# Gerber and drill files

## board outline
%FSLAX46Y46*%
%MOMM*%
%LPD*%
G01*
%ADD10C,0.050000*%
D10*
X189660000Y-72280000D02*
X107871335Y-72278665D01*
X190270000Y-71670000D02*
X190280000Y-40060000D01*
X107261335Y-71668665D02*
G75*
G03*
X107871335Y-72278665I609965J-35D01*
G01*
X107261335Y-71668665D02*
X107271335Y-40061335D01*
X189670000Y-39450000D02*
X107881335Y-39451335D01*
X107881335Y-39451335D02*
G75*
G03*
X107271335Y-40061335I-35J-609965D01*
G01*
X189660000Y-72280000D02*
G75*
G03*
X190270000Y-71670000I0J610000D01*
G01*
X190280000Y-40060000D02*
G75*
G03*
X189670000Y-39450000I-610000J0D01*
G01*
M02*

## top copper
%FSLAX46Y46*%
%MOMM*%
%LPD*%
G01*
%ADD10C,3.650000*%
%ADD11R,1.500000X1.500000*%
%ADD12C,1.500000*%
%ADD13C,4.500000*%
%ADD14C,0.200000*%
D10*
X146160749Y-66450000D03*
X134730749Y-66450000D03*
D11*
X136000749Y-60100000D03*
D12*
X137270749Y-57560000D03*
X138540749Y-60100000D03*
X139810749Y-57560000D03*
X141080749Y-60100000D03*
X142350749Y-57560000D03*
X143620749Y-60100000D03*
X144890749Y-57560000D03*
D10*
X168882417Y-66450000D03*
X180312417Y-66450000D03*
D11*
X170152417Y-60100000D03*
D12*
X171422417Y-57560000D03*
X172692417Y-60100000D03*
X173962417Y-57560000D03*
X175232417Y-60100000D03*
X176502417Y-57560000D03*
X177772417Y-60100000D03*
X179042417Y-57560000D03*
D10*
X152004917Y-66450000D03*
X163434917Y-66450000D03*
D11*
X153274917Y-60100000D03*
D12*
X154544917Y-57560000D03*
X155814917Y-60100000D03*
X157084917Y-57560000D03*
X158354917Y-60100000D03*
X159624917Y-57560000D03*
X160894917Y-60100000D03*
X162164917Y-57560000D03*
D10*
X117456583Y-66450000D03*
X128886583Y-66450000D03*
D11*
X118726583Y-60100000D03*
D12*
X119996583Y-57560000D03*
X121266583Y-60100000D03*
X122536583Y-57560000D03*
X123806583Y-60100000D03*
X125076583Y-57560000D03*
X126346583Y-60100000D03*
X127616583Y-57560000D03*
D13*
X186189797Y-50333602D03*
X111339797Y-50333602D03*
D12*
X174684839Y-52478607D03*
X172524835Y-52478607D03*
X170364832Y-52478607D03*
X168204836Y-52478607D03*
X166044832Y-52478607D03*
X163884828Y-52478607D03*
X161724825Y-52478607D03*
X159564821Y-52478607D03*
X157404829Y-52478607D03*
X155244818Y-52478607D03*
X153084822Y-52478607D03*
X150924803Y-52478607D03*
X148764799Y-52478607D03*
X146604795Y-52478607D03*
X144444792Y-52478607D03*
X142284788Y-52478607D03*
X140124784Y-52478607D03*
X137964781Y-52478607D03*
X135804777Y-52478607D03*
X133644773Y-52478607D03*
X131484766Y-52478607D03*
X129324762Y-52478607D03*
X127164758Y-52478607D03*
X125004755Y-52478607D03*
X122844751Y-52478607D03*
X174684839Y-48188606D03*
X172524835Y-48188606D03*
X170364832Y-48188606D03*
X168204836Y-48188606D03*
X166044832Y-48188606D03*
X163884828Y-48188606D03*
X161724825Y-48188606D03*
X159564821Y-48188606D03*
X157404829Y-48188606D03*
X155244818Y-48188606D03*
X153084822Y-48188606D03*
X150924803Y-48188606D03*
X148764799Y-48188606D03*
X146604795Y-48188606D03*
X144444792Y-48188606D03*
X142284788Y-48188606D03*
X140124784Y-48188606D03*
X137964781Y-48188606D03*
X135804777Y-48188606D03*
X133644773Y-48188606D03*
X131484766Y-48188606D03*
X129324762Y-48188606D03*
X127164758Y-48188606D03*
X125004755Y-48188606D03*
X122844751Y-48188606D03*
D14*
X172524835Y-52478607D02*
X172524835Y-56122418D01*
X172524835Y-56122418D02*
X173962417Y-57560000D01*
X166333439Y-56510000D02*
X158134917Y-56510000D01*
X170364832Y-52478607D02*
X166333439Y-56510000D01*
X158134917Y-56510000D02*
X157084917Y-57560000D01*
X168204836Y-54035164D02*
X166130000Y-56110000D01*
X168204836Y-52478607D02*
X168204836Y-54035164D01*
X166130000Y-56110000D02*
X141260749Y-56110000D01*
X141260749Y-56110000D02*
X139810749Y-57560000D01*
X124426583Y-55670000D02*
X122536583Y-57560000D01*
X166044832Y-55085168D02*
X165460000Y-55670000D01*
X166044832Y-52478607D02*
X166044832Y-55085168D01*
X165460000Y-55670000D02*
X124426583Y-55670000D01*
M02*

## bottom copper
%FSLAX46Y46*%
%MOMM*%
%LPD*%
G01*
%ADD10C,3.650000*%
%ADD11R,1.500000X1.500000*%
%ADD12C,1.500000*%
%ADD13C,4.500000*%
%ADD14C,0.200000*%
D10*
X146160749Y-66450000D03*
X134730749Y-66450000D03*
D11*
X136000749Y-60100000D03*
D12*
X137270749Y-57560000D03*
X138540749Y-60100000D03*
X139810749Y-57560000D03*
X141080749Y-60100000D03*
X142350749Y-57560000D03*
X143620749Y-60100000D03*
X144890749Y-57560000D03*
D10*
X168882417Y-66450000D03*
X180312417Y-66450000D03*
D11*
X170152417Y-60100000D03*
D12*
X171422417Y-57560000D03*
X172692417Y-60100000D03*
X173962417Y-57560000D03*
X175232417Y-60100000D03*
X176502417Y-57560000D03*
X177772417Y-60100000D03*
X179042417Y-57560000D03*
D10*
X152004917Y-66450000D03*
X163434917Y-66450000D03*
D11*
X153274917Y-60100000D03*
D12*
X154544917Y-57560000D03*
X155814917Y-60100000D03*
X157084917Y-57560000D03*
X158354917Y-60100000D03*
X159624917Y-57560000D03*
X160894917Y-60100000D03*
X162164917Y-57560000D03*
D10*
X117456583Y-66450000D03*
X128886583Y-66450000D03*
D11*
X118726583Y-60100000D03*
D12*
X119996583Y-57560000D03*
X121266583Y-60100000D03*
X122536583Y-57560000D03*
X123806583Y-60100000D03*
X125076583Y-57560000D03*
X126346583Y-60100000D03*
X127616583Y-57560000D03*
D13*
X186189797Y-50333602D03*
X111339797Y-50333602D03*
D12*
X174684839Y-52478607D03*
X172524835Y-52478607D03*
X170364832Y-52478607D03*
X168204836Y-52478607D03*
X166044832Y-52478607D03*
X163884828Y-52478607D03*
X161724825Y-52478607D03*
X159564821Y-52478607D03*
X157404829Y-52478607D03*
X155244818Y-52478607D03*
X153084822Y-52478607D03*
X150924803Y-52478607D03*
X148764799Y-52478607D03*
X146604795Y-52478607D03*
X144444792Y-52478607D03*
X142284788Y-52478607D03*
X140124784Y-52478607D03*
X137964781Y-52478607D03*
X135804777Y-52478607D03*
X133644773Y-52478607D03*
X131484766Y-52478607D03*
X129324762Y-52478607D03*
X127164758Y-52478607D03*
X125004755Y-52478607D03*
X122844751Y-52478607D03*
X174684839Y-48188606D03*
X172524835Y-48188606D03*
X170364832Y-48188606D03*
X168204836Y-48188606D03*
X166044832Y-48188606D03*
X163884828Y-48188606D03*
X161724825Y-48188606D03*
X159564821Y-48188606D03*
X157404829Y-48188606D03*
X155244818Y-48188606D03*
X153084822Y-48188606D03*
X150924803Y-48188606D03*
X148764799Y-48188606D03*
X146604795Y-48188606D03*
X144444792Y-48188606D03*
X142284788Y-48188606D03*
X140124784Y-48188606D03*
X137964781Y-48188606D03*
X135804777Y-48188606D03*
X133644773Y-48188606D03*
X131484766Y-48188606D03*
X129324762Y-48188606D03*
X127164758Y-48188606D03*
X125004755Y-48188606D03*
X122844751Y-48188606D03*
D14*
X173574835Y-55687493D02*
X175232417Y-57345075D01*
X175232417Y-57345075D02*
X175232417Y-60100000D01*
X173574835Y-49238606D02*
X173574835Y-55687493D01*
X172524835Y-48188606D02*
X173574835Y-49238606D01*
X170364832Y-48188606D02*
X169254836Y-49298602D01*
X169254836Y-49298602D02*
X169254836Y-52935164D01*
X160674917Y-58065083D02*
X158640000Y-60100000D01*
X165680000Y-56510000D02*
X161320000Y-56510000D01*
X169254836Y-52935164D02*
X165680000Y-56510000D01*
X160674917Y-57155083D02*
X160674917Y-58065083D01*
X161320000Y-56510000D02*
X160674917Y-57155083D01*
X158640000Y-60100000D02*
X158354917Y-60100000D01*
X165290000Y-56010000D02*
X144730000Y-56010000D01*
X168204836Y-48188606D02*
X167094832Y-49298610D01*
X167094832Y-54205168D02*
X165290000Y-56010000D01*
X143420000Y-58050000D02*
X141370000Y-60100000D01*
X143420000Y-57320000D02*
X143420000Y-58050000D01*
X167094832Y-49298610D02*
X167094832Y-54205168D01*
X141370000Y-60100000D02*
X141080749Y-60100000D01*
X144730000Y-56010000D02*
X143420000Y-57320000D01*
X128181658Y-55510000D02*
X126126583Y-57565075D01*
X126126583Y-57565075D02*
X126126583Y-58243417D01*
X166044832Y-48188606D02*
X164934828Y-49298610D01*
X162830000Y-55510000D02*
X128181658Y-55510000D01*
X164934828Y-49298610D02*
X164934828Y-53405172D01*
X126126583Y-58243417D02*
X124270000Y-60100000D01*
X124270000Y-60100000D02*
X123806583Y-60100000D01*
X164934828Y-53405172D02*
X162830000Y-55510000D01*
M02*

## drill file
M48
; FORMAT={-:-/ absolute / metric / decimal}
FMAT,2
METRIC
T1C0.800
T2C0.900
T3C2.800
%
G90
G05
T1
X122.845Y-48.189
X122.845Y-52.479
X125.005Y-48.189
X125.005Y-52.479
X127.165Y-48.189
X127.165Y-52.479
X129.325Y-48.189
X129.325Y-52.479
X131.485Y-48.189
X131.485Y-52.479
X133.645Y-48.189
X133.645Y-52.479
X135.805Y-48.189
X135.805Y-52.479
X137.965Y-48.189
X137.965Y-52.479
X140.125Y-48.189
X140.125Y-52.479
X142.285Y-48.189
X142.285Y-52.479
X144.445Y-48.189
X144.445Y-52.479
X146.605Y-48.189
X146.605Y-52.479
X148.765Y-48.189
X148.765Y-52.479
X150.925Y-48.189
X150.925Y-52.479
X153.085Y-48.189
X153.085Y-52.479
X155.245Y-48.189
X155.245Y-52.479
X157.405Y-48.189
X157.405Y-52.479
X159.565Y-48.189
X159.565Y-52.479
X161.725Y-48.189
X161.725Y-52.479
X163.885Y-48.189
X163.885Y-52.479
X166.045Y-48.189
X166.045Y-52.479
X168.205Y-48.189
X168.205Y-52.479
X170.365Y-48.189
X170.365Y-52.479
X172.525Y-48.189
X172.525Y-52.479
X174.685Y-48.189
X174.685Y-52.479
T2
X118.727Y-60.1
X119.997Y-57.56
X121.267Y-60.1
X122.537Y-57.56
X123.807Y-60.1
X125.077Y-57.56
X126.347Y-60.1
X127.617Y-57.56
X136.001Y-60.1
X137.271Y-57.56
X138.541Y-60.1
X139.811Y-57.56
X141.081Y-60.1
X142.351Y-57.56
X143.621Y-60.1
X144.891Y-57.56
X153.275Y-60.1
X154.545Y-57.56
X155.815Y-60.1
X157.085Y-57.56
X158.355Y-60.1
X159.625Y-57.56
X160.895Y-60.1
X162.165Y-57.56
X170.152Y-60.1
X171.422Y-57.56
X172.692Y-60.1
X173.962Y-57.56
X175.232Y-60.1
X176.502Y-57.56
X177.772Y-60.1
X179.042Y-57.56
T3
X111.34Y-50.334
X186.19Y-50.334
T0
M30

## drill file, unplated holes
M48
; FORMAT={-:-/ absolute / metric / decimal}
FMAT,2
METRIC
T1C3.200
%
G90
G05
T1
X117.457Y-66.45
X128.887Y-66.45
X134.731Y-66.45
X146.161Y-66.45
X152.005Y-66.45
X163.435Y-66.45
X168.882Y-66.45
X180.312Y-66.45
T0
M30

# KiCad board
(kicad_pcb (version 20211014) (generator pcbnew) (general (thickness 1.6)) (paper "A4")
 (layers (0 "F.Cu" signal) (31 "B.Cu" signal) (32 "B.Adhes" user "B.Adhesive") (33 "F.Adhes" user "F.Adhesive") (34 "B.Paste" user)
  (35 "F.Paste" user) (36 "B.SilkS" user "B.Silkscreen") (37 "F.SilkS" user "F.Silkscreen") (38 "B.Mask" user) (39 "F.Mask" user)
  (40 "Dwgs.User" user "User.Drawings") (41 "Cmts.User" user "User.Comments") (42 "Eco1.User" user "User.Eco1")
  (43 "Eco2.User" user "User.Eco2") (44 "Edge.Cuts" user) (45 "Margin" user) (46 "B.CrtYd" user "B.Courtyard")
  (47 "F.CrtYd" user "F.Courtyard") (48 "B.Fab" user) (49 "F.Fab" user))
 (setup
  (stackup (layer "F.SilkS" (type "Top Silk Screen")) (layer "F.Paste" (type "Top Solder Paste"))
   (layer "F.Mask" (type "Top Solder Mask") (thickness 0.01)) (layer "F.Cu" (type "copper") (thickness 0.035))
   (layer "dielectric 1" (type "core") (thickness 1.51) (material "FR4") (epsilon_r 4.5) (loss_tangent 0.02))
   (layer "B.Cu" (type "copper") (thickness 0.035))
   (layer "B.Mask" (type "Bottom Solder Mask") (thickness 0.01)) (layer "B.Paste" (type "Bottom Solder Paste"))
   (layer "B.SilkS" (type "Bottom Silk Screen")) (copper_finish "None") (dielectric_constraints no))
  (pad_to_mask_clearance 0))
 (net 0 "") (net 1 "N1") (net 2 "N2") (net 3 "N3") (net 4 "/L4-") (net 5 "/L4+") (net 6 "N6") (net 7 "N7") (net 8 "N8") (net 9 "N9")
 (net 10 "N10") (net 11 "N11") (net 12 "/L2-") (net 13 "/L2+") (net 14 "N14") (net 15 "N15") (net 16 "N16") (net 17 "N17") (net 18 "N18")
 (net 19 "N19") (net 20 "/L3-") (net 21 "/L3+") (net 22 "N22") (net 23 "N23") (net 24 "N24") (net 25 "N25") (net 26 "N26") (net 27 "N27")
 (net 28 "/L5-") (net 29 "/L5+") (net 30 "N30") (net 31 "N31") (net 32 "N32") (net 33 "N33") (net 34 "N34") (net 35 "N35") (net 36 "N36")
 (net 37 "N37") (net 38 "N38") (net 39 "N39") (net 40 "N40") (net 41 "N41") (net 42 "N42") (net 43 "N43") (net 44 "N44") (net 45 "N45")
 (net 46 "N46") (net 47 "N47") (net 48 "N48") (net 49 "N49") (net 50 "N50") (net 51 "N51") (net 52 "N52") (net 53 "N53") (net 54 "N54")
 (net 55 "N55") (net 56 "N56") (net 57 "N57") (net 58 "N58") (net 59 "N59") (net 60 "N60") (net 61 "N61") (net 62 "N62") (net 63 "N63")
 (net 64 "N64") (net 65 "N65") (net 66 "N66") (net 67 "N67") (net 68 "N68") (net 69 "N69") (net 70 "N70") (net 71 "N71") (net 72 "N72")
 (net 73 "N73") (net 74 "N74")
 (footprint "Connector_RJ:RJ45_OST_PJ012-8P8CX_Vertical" (layer "F.Cu") (at 136.000749 60.1)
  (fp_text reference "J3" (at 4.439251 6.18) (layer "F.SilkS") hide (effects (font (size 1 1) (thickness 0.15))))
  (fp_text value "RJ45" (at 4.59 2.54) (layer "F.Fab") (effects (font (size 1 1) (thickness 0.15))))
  (pad "" np_thru_hole circle (at 10.16 6.35) (size 3.65 3.65) (drill 3.2) (layers F&B.Cu *.SilkS *.Mask))
  (pad "" np_thru_hole circle (at -1.27 6.35) (size 3.65 3.65) (drill 3.2) (layers F&B.Cu *.SilkS *.Mask))
  (pad "1" thru_hole rect (at 0 0) (size 1.5 1.5) (drill 0.9) (layers *.Cu *.Mask) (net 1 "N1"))
  (pad "2" thru_hole circle (at 1.27 -2.54) (size 1.5 1.5) (drill 0.9) (layers *.Cu *.Mask) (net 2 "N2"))
  (pad "3" thru_hole circle (at 2.54 0) (size 1.5 1.5) (drill 0.9) (layers *.Cu *.Mask) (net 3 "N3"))
  (pad "4" thru_hole circle (at 3.81 -2.54) (size 1.5 1.5) (drill 0.9) (layers *.Cu *.Mask) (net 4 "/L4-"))
  (pad "5" thru_hole circle (at 5.08 0) (size 1.5 1.5) (drill 0.9) (layers *.Cu *.Mask) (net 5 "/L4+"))
  (pad "6" thru_hole circle (at 6.35 -2.54) (size 1.5 1.5) (drill 0.9) (layers *.Cu *.Mask) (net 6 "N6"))
  (pad "7" thru_hole circle (at 7.62 0) (size 1.5 1.5) (drill 0.9) (layers *.Cu *.Mask) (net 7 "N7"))
  (pad "8" thru_hole circle (at 8.89 -2.54) (size 1.5 1.5) (drill 0.9) (layers *.Cu *.Mask) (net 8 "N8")))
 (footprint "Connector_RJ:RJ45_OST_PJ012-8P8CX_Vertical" (layer "F.Cu") (at 170.152417 60.1)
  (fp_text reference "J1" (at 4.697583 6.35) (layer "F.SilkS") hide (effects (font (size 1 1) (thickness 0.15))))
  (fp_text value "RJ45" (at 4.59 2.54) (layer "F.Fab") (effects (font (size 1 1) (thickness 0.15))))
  (pad "" np_thru_hole circle (at -1.27 6.35) (size 3.65 3.65) (drill 3.2) (layers F&B.Cu *.SilkS *.Mask))
  (pad "" np_thru_hole circle (at 10.16 6.35) (size 3.65 3.65) (drill 3.2) (layers F&B.Cu *.SilkS *.Mask))
  (pad "1" thru_hole rect (at 0 0) (size 1.5 1.5) (drill 0.9) (layers *.Cu *.Mask) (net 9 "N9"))
  (pad "2" thru_hole circle (at 1.27 -2.54) (size 1.5 1.5) (drill 0.9) (layers *.Cu *.Mask) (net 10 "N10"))
  (pad "3" thru_hole circle (at 2.54 0) (size 1.5 1.5) (drill 0.9) (layers *.Cu *.Mask) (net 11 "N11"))
  (pad "4" thru_hole circle (at 3.81 -2.54) (size 1.5 1.5) (drill 0.9) (layers *.Cu *.Mask) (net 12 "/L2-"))
  (pad "5" thru_hole circle (at 5.08 0) (size 1.5 1.5) (drill 0.9) (layers *.Cu *.Mask) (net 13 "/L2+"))
  (pad "6" thru_hole circle (at 6.35 -2.54) (size 1.5 1.5) (drill 0.9) (layers *.Cu *.Mask) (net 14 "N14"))
  (pad "7" thru_hole circle (at 7.62 0) (size 1.5 1.5) (drill 0.9) (layers *.Cu *.Mask) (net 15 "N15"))
  (pad "8" thru_hole circle (at 8.89 -2.54) (size 1.5 1.5) (drill 0.9) (layers *.Cu *.Mask) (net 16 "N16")))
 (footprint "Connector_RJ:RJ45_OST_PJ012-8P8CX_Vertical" (layer "F.Cu") (at 153.274917 60.1)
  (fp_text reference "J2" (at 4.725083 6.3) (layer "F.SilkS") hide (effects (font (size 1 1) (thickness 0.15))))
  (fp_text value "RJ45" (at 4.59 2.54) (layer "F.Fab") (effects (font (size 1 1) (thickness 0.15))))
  (pad "" np_thru_hole circle (at -1.27 6.35) (size 3.65 3.65) (drill 3.2) (layers F&B.Cu *.SilkS *.Mask))
  (pad "" np_thru_hole circle (at 10.16 6.35) (size 3.65 3.65) (drill 3.2) (layers F&B.Cu *.SilkS *.Mask))
  (pad "1" thru_hole rect (at 0 0) (size 1.5 1.5) (drill 0.9) (layers *.Cu *.Mask) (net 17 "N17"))
  (pad "2" thru_hole circle (at 1.27 -2.54) (size 1.5 1.5) (drill 0.9) (layers *.Cu *.Mask) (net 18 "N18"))
  (pad "3" thru_hole circle (at 2.54 0) (size 1.5 1.5) (drill 0.9) (layers *.Cu *.Mask) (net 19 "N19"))
  (pad "4" thru_hole circle (at 3.81 -2.54) (size 1.5 1.5) (drill 0.9) (layers *.Cu *.Mask) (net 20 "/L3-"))
  (pad "5" thru_hole circle (at 5.08 0) (size 1.5 1.5) (drill 0.9) (layers *.Cu *.Mask) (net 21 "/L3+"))
  (pad "6" thru_hole circle (at 6.35 -2.54) (size 1.5 1.5) (drill 0.9) (layers *.Cu *.Mask) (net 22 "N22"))
  (pad "7" thru_hole circle (at 7.62 0) (size 1.5 1.5) (drill 0.9) (layers *.Cu *.Mask) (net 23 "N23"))
  (pad "8" thru_hole circle (at 8.89 -2.54) (size 1.5 1.5) (drill 0.9) (layers *.Cu *.Mask) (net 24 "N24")))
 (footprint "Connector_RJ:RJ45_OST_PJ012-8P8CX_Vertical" (layer "F.Cu") (at 118.726583 60.1)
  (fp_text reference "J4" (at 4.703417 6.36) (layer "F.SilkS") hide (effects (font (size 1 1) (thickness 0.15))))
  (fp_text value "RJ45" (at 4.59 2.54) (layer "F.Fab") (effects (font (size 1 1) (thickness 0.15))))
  (pad "" np_thru_hole circle (at -1.27 6.35) (size 3.65 3.65) (drill 3.2) (layers F&B.Cu *.SilkS *.Mask))
  (pad "" np_thru_hole circle (at 10.16 6.35) (size 3.65 3.65) (drill 3.2) (layers F&B.Cu *.SilkS *.Mask))
  (pad "1" thru_hole rect (at 0 0) (size 1.5 1.5) (drill 0.9) (layers *.Cu *.Mask) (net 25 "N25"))
  (pad "2" thru_hole circle (at 1.27 -2.54) (size 1.5 1.5) (drill 0.9) (layers *.Cu *.Mask) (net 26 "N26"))
  (pad "3" thru_hole circle (at 2.54 0) (size 1.5 1.5) (drill 0.9) (layers *.Cu *.Mask) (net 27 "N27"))
  (pad "4" thru_hole circle (at 3.81 -2.54) (size 1.5 1.5) (drill 0.9) (layers *.Cu *.Mask) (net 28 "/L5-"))
  (pad "5" thru_hole circle (at 5.08 0) (size 1.5 1.5) (drill 0.9) (layers *.Cu *.Mask) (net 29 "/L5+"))
  (pad "6" thru_hole circle (at 6.35 -2.54) (size 1.5 1.5) (drill 0.9) (layers *.Cu *.Mask) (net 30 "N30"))
  (pad "7" thru_hole circle (at 7.62 0) (size 1.5 1.5) (drill 0.9) (layers *.Cu *.Mask) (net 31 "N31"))
  (pad "8" thru_hole circle (at 8.89 -2.54) (size 1.5 1.5) (drill 0.9) (layers *.Cu *.Mask) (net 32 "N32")))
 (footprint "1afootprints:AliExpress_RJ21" (layer "F.Cu") (at 149.8 46.9)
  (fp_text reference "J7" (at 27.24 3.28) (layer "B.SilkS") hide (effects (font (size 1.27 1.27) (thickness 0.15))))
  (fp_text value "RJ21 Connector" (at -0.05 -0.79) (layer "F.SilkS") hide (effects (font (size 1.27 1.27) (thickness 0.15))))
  (pad "" thru_hole circle locked (at 36.389797 3.433602) (size 4.5 4.5) (drill 2.8) (layers *.Cu *.Mask))
  (pad "" thru_hole circle locked (at -38.460203 3.433602) (size 4.5 4.5) (drill 2.8) (layers *.Cu *.Mask))
  (pad "1" thru_hole circle locked (at 24.884839 5.578607) (size 1.5 1.5) (drill 0.8) (layers *.Cu *.Mask) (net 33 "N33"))
  (pad "2" thru_hole circle locked (at 22.724835 5.578607) (size 1.5 1.5) (drill 0.8) (layers *.Cu *.Mask) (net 12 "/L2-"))
  (pad "3" thru_hole circle locked (at 20.564832 5.578607) (size 1.5 1.5) (drill 0.8) (layers *.Cu *.Mask) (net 20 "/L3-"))
  (pad "4" thru_hole circle locked (at 18.404836 5.578607) (size 1.5 1.5) (drill 0.8) (layers *.Cu *.Mask) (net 4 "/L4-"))
  (pad "5" thru_hole circle locked (at 16.244832 5.578607) (size 1.5 1.5) (drill 0.8) (layers *.Cu *.Mask) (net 28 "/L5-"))
  (pad "6" thru_hole circle locked (at 14.084828 5.578607) (size 1.5 1.5) (drill 0.8) (layers *.Cu *.Mask) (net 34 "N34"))
  (pad "7" thru_hole circle locked (at 11.924825 5.578607) (size 1.5 1.5) (drill 0.8) (layers *.Cu *.Mask) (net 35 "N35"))
  (pad "8" thru_hole circle locked (at 9.764821 5.578607) (size 1.5 1.5) (drill 0.8) (layers *.Cu *.Mask) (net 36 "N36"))
  (pad "9" thru_hole circle locked (at 7.604829 5.578607) (size 1.5 1.5) (drill 0.8) (layers *.Cu *.Mask) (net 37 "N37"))
  (pad "10" thru_hole circle locked (at 5.444818 5.578607) (size 1.5 1.5) (drill 0.8) (layers *.Cu *.Mask) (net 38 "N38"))
  (pad "11" thru_hole circle locked (at 3.284822 5.578607) (size 1.5 1.5) (drill 0.8) (layers *.Cu *.Mask) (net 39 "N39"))
  (pad "12" thru_hole circle locked (at 1.124803 5.578607) (size 1.5 1.5) (drill 0.8) (layers *.Cu *.Mask) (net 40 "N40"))
  (pad "13" thru_hole circle locked (at -1.035201 5.578607) (size 1.5 1.5) (drill 0.8) (layers *.Cu *.Mask) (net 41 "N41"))
  (pad "14" thru_hole circle locked (at -3.195205 5.578607) (size 1.5 1.5) (drill 0.8) (layers *.Cu *.Mask) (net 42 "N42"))
  (pad "15" thru_hole circle locked (at -5.355208 5.578607) (size 1.5 1.5) (drill 0.8) (layers *.Cu *.Mask) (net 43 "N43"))
  (pad "16" thru_hole circle locked (at -7.515212 5.578607) (size 1.5 1.5) (drill 0.8) (layers *.Cu *.Mask) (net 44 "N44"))
  (pad "17" thru_hole circle locked (at -9.675216 5.578607) (size 1.5 1.5) (drill 0.8) (layers *.Cu *.Mask) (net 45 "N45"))
  (pad "18" thru_hole circle locked (at -11.835219 5.578607) (size 1.5 1.5) (drill 0.8) (layers *.Cu *.Mask) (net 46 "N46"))
  (pad "19" thru_hole circle locked (at -13.995223 5.578607) (size 1.5 1.5) (drill 0.8) (layers *.Cu *.Mask) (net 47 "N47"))
  (pad "20" thru_hole circle locked (at -16.155227 5.578607) (size 1.5 1.5) (drill 0.8) (layers *.Cu *.Mask) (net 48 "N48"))
  (pad "21" thru_hole circle locked (at -18.315234 5.578607) (size 1.5 1.5) (drill 0.8) (layers *.Cu *.Mask) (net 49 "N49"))
  (pad "22" thru_hole circle locked (at -20.475238 5.578607) (size 1.5 1.5) (drill 0.8) (layers *.Cu *.Mask) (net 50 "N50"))
  (pad "23" thru_hole circle locked (at -22.635242 5.578607) (size 1.5 1.5) (drill 0.8) (layers *.Cu *.Mask) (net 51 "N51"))
  (pad "24" thru_hole circle locked (at -24.795245 5.578607) (size 1.5 1.5) (drill 0.8) (layers *.Cu *.Mask) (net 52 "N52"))
  (pad "25" thru_hole circle locked (at -26.955249 5.578607) (size 1.5 1.5) (drill 0.8) (layers *.Cu *.Mask) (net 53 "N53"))
  (pad "26" thru_hole circle locked (at 24.884839 1.288606) (size 1.5 1.5) (drill 0.8) (layers *.Cu *.Mask) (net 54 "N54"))
  (pad "27" thru_hole circle locked (at 22.724835 1.288606) (size 1.5 1.5) (drill 0.8) (layers *.Cu *.Mask) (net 13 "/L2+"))
  (pad "28" thru_hole circle locked (at 20.564832 1.288606) (size 1.5 1.5) (drill 0.8) (layers *.Cu *.Mask) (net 21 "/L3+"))
  (pad "29" thru_hole circle locked (at 18.404836 1.288606) (size 1.5 1.5) (drill 0.8) (layers *.Cu *.Mask) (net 5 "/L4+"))
  (pad "30" thru_hole circle locked (at 16.244832 1.288606) (size 1.5 1.5) (drill 0.8) (layers *.Cu *.Mask) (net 29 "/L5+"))
  (pad "31" thru_hole circle locked (at 14.084828 1.288606) (size 1.5 1.5) (drill 0.8) (layers *.Cu *.Mask) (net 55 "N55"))
  (pad "32" thru_hole circle locked (at 11.924825 1.288606) (size 1.5 1.5) (drill 0.8) (layers *.Cu *.Mask) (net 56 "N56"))
  (pad "33" thru_hole circle locked (at 9.764821 1.288606) (size 1.5 1.5) (drill 0.8) (layers *.Cu *.Mask) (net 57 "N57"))
  (pad "34" thru_hole circle locked (at 7.604829 1.288606) (size 1.5 1.5) (drill 0.8) (layers *.Cu *.Mask) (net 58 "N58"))
  (pad "35" thru_hole circle locked (at 5.444818 1.288606) (size 1.5 1.5) (drill 0.8) (layers *.Cu *.Mask) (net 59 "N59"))
  (pad "36" thru_hole circle locked (at 3.284822 1.288606) (size 1.5 1.5) (drill 0.8) (layers *.Cu *.Mask) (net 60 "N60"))
  (pad "37" thru_hole circle locked (at 1.124803 1.288606) (size 1.5 1.5) (drill 0.8) (layers *.Cu *.Mask) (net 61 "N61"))
  (pad "38" thru_hole circle locked (at -1.035201 1.288606) (size 1.5 1.5) (drill 0.8) (layers *.Cu *.Mask) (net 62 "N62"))
  (pad "39" thru_hole circle locked (at -3.195205 1.288606) (size 1.5 1.5) (drill 0.8) (layers *.Cu *.Mask) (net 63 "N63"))
  (pad "40" thru_hole circle locked (at -5.355208 1.288606) (size 1.5 1.5) (drill 0.8) (layers *.Cu *.Mask) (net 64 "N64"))
  (pad "41" thru_hole circle locked (at -7.515212 1.288606) (size 1.5 1.5) (drill 0.8) (layers *.Cu *.Mask) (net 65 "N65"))
  (pad "42" thru_hole circle locked (at -9.675216 1.288606) (size 1.5 1.5) (drill 0.8) (layers *.Cu *.Mask) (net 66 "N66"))
  (pad "43" thru_hole circle locked (at -11.835219 1.288606) (size 1.5 1.5) (drill 0.8) (layers *.Cu *.Mask) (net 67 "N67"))
  (pad "44" thru_hole circle locked (at -13.995223 1.288606) (size 1.5 1.5) (drill 0.8) (layers *.Cu *.Mask) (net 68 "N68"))
  (pad "45" thru_hole circle locked (at -16.155227 1.288606) (size 1.5 1.5) (drill 0.8) (layers *.Cu *.Mask) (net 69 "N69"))
  (pad "46" thru_hole circle locked (at -18.315234 1.288606) (size 1.5 1.5) (drill 0.8) (layers *.Cu *.Mask) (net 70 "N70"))
  (pad "47" thru_hole circle locked (at -20.475238 1.288606) (size 1.5 1.5) (drill 0.8) (layers *.Cu *.Mask) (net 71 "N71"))
  (pad "48" thru_hole circle locked (at -22.635242 1.288606) (size 1.5 1.5) (drill 0.8) (layers *.Cu *.Mask) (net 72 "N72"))
  (pad "49" thru_hole circle locked (at -24.795245 1.288606) (size 1.5 1.5) (drill 0.8) (layers *.Cu *.Mask) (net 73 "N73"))
  (pad "50" thru_hole circle locked (at -26.955249 1.288606) (size 1.5 1.5) (drill 0.8) (layers *.Cu *.Mask) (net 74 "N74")))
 (gr_line (start 189.66 72.28) (end 107.871335 72.278665) (layer "Edge.Cuts") (width 0.05))
 (gr_line (start 190.27 71.67) (end 190.28 40.06) (layer "Edge.Cuts") (width 0.05))
 (gr_arc (start 107.871335 72.278665) (mid 107.44 72.1) (end 107.261335 71.668665) (layer "Edge.Cuts") (width 0.05))
 (gr_line (start 107.261335 71.668665) (end 107.271335 40.061335) (layer "Edge.Cuts") (width 0.05))
 (gr_line (start 189.67 39.45) (end 107.881335 39.451335) (layer "Edge.Cuts") (width 0.05))
 (gr_arc (start 107.271335 40.061335) (mid 107.45 39.63) (end 107.881335 39.451335) (layer "Edge.Cuts") (width 0.05))
 (gr_arc (start 190.27 71.67) (mid 190.091335 72.101335) (end 189.66 72.28) (layer "Edge.Cuts") (width 0.05))
 (gr_arc (start 189.67 39.45) (mid 190.101335 39.628665) (end 190.28 40.06) (layer "Edge.Cuts") (width 0.05))
 (segment (start 173.574835 55.687493) (end 175.232417 57.345075) (width 0.2) (layer "B.Cu") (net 13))
 (segment (start 175.232417 57.345075) (end 175.232417 60.1) (width 0.2) (layer "B.Cu") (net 13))
 (segment (start 173.574835 49.238606) (end 173.574835 55.687493) (width 0.2) (layer "B.Cu") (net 13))
 (segment (start 172.524835 48.188606) (end 173.574835 49.238606) (width 0.2) (layer "B.Cu") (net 13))
 (segment (start 172.524835 52.478607) (end 172.524835 56.122418) (width 0.2) (layer "F.Cu") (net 12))
 (segment (start 172.524835 56.122418) (end 173.962417 57.56) (width 0.2) (layer "F.Cu") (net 12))
 (segment (start 166.333439 56.51) (end 158.134917 56.51) (width 0.2) (layer "F.Cu") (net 20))
 (segment (start 170.364832 52.478607) (end 166.333439 56.51) (width 0.2) (layer "F.Cu") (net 20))
 (segment (start 158.134917 56.51) (end 157.084917 57.56) (width 0.2) (layer "F.Cu") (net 20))
 (segment (start 170.364832 48.188606) (end 169.254836 49.298602) (width 0.2) (layer "B.Cu") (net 21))
 (segment (start 169.254836 49.298602) (end 169.254836 52.935164) (width 0.2) (layer "B.Cu") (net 21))
 (segment (start 160.674917 58.065083) (end 158.64 60.1) (width 0.2) (layer "B.Cu") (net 21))
 (segment (start 165.68 56.51) (end 161.32 56.51) (width 0.2) (layer "B.Cu") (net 21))
 (segment (start 169.254836 52.935164) (end 165.68 56.51) (width 0.2) (layer "B.Cu") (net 21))
 (segment (start 160.674917 57.155083) (end 160.674917 58.065083) (width 0.2) (layer "B.Cu") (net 21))
 (segment (start 161.32 56.51) (end 160.674917 57.155083) (width 0.2) (layer "B.Cu") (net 21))
 (segment (start 158.64 60.1) (end 158.354917 60.1) (width 0.2) (layer "B.Cu") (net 21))
 (segment (start 165.29 56.01) (end 144.73 56.01) (width 0.2) (layer "B.Cu") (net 5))
 (segment (start 168.204836 48.188606) (end 167.094832 49.29861) (width 0.2) (layer "B.Cu") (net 5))
 (segment (start 167.094832 54.205168) (end 165.29 56.01) (width 0.2) (layer "B.Cu") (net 5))
 (segment (start 143.42 58.05) (end 141.37 60.1) (width 0.2) (layer "B.Cu") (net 5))
 (segment (start 143.42 57.32) (end 143.42 58.05) (width 0.2) (layer "B.Cu") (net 5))
 (segment (start 167.094832 49.29861) (end 167.094832 54.205168) (width 0.2) (layer "B.Cu") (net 5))
 (segment (start 141.37 60.1) (end 141.080749 60.1) (width 0.2) (layer "B.Cu") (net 5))
 (segment (start 144.73 56.01) (end 143.42 57.32) (width 0.2) (layer "B.Cu") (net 5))
 (segment (start 168.204836 54.035164) (end 166.13 56.11) (width 0.2) (layer "F.Cu") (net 4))
 (segment (start 168.204836 52.478607) (end 168.204836 54.035164) (width 0.2) (layer "F.Cu") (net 4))
 (segment (start 166.13 56.11) (end 141.260749 56.11) (width 0.2) (layer "F.Cu") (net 4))
 (segment (start 141.260749 56.11) (end 139.810749 57.56) (width 0.2) (layer "F.Cu") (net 4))
 (segment (start 124.426583 55.67) (end 122.536583 57.56) (width 0.2) (layer "F.Cu") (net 28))
 (segment (start 166.044832 55.085168) (end 165.46 55.67) (width 0.2) (layer "F.Cu") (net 28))
 (segment (start 166.044832 52.478607) (end 166.044832 55.085168) (width 0.2) (layer "F.Cu") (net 28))
 (segment (start 165.46 55.67) (end 124.426583 55.67) (width 0.2) (layer "F.Cu") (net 28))
 (segment (start 128.181658 55.51) (end 126.126583 57.565075) (width 0.2) (layer "B.Cu") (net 29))
 (segment (start 126.126583 57.565075) (end 126.126583 58.243417) (width 0.2) (layer "B.Cu") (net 29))
 (segment (start 166.044832 48.188606) (end 164.934828 49.29861) (width 0.2) (layer "B.Cu") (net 29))
 (segment (start 162.83 55.51) (end 128.181658 55.51) (width 0.2) (layer "B.Cu") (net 29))
 (segment (start 164.934828 49.29861) (end 164.934828 53.405172) (width 0.2) (layer "B.Cu") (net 29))
 (segment (start 126.126583 58.243417) (end 124.27 60.1) (width 0.2) (layer "B.Cu") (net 29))
 (segment (start 124.27 60.1) (end 123.806583 60.1) (width 0.2) (layer "B.Cu") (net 29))
 (segment (start 164.934828 53.405172) (end 162.83 55.51) (width 0.2) (layer "B.Cu") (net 29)))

